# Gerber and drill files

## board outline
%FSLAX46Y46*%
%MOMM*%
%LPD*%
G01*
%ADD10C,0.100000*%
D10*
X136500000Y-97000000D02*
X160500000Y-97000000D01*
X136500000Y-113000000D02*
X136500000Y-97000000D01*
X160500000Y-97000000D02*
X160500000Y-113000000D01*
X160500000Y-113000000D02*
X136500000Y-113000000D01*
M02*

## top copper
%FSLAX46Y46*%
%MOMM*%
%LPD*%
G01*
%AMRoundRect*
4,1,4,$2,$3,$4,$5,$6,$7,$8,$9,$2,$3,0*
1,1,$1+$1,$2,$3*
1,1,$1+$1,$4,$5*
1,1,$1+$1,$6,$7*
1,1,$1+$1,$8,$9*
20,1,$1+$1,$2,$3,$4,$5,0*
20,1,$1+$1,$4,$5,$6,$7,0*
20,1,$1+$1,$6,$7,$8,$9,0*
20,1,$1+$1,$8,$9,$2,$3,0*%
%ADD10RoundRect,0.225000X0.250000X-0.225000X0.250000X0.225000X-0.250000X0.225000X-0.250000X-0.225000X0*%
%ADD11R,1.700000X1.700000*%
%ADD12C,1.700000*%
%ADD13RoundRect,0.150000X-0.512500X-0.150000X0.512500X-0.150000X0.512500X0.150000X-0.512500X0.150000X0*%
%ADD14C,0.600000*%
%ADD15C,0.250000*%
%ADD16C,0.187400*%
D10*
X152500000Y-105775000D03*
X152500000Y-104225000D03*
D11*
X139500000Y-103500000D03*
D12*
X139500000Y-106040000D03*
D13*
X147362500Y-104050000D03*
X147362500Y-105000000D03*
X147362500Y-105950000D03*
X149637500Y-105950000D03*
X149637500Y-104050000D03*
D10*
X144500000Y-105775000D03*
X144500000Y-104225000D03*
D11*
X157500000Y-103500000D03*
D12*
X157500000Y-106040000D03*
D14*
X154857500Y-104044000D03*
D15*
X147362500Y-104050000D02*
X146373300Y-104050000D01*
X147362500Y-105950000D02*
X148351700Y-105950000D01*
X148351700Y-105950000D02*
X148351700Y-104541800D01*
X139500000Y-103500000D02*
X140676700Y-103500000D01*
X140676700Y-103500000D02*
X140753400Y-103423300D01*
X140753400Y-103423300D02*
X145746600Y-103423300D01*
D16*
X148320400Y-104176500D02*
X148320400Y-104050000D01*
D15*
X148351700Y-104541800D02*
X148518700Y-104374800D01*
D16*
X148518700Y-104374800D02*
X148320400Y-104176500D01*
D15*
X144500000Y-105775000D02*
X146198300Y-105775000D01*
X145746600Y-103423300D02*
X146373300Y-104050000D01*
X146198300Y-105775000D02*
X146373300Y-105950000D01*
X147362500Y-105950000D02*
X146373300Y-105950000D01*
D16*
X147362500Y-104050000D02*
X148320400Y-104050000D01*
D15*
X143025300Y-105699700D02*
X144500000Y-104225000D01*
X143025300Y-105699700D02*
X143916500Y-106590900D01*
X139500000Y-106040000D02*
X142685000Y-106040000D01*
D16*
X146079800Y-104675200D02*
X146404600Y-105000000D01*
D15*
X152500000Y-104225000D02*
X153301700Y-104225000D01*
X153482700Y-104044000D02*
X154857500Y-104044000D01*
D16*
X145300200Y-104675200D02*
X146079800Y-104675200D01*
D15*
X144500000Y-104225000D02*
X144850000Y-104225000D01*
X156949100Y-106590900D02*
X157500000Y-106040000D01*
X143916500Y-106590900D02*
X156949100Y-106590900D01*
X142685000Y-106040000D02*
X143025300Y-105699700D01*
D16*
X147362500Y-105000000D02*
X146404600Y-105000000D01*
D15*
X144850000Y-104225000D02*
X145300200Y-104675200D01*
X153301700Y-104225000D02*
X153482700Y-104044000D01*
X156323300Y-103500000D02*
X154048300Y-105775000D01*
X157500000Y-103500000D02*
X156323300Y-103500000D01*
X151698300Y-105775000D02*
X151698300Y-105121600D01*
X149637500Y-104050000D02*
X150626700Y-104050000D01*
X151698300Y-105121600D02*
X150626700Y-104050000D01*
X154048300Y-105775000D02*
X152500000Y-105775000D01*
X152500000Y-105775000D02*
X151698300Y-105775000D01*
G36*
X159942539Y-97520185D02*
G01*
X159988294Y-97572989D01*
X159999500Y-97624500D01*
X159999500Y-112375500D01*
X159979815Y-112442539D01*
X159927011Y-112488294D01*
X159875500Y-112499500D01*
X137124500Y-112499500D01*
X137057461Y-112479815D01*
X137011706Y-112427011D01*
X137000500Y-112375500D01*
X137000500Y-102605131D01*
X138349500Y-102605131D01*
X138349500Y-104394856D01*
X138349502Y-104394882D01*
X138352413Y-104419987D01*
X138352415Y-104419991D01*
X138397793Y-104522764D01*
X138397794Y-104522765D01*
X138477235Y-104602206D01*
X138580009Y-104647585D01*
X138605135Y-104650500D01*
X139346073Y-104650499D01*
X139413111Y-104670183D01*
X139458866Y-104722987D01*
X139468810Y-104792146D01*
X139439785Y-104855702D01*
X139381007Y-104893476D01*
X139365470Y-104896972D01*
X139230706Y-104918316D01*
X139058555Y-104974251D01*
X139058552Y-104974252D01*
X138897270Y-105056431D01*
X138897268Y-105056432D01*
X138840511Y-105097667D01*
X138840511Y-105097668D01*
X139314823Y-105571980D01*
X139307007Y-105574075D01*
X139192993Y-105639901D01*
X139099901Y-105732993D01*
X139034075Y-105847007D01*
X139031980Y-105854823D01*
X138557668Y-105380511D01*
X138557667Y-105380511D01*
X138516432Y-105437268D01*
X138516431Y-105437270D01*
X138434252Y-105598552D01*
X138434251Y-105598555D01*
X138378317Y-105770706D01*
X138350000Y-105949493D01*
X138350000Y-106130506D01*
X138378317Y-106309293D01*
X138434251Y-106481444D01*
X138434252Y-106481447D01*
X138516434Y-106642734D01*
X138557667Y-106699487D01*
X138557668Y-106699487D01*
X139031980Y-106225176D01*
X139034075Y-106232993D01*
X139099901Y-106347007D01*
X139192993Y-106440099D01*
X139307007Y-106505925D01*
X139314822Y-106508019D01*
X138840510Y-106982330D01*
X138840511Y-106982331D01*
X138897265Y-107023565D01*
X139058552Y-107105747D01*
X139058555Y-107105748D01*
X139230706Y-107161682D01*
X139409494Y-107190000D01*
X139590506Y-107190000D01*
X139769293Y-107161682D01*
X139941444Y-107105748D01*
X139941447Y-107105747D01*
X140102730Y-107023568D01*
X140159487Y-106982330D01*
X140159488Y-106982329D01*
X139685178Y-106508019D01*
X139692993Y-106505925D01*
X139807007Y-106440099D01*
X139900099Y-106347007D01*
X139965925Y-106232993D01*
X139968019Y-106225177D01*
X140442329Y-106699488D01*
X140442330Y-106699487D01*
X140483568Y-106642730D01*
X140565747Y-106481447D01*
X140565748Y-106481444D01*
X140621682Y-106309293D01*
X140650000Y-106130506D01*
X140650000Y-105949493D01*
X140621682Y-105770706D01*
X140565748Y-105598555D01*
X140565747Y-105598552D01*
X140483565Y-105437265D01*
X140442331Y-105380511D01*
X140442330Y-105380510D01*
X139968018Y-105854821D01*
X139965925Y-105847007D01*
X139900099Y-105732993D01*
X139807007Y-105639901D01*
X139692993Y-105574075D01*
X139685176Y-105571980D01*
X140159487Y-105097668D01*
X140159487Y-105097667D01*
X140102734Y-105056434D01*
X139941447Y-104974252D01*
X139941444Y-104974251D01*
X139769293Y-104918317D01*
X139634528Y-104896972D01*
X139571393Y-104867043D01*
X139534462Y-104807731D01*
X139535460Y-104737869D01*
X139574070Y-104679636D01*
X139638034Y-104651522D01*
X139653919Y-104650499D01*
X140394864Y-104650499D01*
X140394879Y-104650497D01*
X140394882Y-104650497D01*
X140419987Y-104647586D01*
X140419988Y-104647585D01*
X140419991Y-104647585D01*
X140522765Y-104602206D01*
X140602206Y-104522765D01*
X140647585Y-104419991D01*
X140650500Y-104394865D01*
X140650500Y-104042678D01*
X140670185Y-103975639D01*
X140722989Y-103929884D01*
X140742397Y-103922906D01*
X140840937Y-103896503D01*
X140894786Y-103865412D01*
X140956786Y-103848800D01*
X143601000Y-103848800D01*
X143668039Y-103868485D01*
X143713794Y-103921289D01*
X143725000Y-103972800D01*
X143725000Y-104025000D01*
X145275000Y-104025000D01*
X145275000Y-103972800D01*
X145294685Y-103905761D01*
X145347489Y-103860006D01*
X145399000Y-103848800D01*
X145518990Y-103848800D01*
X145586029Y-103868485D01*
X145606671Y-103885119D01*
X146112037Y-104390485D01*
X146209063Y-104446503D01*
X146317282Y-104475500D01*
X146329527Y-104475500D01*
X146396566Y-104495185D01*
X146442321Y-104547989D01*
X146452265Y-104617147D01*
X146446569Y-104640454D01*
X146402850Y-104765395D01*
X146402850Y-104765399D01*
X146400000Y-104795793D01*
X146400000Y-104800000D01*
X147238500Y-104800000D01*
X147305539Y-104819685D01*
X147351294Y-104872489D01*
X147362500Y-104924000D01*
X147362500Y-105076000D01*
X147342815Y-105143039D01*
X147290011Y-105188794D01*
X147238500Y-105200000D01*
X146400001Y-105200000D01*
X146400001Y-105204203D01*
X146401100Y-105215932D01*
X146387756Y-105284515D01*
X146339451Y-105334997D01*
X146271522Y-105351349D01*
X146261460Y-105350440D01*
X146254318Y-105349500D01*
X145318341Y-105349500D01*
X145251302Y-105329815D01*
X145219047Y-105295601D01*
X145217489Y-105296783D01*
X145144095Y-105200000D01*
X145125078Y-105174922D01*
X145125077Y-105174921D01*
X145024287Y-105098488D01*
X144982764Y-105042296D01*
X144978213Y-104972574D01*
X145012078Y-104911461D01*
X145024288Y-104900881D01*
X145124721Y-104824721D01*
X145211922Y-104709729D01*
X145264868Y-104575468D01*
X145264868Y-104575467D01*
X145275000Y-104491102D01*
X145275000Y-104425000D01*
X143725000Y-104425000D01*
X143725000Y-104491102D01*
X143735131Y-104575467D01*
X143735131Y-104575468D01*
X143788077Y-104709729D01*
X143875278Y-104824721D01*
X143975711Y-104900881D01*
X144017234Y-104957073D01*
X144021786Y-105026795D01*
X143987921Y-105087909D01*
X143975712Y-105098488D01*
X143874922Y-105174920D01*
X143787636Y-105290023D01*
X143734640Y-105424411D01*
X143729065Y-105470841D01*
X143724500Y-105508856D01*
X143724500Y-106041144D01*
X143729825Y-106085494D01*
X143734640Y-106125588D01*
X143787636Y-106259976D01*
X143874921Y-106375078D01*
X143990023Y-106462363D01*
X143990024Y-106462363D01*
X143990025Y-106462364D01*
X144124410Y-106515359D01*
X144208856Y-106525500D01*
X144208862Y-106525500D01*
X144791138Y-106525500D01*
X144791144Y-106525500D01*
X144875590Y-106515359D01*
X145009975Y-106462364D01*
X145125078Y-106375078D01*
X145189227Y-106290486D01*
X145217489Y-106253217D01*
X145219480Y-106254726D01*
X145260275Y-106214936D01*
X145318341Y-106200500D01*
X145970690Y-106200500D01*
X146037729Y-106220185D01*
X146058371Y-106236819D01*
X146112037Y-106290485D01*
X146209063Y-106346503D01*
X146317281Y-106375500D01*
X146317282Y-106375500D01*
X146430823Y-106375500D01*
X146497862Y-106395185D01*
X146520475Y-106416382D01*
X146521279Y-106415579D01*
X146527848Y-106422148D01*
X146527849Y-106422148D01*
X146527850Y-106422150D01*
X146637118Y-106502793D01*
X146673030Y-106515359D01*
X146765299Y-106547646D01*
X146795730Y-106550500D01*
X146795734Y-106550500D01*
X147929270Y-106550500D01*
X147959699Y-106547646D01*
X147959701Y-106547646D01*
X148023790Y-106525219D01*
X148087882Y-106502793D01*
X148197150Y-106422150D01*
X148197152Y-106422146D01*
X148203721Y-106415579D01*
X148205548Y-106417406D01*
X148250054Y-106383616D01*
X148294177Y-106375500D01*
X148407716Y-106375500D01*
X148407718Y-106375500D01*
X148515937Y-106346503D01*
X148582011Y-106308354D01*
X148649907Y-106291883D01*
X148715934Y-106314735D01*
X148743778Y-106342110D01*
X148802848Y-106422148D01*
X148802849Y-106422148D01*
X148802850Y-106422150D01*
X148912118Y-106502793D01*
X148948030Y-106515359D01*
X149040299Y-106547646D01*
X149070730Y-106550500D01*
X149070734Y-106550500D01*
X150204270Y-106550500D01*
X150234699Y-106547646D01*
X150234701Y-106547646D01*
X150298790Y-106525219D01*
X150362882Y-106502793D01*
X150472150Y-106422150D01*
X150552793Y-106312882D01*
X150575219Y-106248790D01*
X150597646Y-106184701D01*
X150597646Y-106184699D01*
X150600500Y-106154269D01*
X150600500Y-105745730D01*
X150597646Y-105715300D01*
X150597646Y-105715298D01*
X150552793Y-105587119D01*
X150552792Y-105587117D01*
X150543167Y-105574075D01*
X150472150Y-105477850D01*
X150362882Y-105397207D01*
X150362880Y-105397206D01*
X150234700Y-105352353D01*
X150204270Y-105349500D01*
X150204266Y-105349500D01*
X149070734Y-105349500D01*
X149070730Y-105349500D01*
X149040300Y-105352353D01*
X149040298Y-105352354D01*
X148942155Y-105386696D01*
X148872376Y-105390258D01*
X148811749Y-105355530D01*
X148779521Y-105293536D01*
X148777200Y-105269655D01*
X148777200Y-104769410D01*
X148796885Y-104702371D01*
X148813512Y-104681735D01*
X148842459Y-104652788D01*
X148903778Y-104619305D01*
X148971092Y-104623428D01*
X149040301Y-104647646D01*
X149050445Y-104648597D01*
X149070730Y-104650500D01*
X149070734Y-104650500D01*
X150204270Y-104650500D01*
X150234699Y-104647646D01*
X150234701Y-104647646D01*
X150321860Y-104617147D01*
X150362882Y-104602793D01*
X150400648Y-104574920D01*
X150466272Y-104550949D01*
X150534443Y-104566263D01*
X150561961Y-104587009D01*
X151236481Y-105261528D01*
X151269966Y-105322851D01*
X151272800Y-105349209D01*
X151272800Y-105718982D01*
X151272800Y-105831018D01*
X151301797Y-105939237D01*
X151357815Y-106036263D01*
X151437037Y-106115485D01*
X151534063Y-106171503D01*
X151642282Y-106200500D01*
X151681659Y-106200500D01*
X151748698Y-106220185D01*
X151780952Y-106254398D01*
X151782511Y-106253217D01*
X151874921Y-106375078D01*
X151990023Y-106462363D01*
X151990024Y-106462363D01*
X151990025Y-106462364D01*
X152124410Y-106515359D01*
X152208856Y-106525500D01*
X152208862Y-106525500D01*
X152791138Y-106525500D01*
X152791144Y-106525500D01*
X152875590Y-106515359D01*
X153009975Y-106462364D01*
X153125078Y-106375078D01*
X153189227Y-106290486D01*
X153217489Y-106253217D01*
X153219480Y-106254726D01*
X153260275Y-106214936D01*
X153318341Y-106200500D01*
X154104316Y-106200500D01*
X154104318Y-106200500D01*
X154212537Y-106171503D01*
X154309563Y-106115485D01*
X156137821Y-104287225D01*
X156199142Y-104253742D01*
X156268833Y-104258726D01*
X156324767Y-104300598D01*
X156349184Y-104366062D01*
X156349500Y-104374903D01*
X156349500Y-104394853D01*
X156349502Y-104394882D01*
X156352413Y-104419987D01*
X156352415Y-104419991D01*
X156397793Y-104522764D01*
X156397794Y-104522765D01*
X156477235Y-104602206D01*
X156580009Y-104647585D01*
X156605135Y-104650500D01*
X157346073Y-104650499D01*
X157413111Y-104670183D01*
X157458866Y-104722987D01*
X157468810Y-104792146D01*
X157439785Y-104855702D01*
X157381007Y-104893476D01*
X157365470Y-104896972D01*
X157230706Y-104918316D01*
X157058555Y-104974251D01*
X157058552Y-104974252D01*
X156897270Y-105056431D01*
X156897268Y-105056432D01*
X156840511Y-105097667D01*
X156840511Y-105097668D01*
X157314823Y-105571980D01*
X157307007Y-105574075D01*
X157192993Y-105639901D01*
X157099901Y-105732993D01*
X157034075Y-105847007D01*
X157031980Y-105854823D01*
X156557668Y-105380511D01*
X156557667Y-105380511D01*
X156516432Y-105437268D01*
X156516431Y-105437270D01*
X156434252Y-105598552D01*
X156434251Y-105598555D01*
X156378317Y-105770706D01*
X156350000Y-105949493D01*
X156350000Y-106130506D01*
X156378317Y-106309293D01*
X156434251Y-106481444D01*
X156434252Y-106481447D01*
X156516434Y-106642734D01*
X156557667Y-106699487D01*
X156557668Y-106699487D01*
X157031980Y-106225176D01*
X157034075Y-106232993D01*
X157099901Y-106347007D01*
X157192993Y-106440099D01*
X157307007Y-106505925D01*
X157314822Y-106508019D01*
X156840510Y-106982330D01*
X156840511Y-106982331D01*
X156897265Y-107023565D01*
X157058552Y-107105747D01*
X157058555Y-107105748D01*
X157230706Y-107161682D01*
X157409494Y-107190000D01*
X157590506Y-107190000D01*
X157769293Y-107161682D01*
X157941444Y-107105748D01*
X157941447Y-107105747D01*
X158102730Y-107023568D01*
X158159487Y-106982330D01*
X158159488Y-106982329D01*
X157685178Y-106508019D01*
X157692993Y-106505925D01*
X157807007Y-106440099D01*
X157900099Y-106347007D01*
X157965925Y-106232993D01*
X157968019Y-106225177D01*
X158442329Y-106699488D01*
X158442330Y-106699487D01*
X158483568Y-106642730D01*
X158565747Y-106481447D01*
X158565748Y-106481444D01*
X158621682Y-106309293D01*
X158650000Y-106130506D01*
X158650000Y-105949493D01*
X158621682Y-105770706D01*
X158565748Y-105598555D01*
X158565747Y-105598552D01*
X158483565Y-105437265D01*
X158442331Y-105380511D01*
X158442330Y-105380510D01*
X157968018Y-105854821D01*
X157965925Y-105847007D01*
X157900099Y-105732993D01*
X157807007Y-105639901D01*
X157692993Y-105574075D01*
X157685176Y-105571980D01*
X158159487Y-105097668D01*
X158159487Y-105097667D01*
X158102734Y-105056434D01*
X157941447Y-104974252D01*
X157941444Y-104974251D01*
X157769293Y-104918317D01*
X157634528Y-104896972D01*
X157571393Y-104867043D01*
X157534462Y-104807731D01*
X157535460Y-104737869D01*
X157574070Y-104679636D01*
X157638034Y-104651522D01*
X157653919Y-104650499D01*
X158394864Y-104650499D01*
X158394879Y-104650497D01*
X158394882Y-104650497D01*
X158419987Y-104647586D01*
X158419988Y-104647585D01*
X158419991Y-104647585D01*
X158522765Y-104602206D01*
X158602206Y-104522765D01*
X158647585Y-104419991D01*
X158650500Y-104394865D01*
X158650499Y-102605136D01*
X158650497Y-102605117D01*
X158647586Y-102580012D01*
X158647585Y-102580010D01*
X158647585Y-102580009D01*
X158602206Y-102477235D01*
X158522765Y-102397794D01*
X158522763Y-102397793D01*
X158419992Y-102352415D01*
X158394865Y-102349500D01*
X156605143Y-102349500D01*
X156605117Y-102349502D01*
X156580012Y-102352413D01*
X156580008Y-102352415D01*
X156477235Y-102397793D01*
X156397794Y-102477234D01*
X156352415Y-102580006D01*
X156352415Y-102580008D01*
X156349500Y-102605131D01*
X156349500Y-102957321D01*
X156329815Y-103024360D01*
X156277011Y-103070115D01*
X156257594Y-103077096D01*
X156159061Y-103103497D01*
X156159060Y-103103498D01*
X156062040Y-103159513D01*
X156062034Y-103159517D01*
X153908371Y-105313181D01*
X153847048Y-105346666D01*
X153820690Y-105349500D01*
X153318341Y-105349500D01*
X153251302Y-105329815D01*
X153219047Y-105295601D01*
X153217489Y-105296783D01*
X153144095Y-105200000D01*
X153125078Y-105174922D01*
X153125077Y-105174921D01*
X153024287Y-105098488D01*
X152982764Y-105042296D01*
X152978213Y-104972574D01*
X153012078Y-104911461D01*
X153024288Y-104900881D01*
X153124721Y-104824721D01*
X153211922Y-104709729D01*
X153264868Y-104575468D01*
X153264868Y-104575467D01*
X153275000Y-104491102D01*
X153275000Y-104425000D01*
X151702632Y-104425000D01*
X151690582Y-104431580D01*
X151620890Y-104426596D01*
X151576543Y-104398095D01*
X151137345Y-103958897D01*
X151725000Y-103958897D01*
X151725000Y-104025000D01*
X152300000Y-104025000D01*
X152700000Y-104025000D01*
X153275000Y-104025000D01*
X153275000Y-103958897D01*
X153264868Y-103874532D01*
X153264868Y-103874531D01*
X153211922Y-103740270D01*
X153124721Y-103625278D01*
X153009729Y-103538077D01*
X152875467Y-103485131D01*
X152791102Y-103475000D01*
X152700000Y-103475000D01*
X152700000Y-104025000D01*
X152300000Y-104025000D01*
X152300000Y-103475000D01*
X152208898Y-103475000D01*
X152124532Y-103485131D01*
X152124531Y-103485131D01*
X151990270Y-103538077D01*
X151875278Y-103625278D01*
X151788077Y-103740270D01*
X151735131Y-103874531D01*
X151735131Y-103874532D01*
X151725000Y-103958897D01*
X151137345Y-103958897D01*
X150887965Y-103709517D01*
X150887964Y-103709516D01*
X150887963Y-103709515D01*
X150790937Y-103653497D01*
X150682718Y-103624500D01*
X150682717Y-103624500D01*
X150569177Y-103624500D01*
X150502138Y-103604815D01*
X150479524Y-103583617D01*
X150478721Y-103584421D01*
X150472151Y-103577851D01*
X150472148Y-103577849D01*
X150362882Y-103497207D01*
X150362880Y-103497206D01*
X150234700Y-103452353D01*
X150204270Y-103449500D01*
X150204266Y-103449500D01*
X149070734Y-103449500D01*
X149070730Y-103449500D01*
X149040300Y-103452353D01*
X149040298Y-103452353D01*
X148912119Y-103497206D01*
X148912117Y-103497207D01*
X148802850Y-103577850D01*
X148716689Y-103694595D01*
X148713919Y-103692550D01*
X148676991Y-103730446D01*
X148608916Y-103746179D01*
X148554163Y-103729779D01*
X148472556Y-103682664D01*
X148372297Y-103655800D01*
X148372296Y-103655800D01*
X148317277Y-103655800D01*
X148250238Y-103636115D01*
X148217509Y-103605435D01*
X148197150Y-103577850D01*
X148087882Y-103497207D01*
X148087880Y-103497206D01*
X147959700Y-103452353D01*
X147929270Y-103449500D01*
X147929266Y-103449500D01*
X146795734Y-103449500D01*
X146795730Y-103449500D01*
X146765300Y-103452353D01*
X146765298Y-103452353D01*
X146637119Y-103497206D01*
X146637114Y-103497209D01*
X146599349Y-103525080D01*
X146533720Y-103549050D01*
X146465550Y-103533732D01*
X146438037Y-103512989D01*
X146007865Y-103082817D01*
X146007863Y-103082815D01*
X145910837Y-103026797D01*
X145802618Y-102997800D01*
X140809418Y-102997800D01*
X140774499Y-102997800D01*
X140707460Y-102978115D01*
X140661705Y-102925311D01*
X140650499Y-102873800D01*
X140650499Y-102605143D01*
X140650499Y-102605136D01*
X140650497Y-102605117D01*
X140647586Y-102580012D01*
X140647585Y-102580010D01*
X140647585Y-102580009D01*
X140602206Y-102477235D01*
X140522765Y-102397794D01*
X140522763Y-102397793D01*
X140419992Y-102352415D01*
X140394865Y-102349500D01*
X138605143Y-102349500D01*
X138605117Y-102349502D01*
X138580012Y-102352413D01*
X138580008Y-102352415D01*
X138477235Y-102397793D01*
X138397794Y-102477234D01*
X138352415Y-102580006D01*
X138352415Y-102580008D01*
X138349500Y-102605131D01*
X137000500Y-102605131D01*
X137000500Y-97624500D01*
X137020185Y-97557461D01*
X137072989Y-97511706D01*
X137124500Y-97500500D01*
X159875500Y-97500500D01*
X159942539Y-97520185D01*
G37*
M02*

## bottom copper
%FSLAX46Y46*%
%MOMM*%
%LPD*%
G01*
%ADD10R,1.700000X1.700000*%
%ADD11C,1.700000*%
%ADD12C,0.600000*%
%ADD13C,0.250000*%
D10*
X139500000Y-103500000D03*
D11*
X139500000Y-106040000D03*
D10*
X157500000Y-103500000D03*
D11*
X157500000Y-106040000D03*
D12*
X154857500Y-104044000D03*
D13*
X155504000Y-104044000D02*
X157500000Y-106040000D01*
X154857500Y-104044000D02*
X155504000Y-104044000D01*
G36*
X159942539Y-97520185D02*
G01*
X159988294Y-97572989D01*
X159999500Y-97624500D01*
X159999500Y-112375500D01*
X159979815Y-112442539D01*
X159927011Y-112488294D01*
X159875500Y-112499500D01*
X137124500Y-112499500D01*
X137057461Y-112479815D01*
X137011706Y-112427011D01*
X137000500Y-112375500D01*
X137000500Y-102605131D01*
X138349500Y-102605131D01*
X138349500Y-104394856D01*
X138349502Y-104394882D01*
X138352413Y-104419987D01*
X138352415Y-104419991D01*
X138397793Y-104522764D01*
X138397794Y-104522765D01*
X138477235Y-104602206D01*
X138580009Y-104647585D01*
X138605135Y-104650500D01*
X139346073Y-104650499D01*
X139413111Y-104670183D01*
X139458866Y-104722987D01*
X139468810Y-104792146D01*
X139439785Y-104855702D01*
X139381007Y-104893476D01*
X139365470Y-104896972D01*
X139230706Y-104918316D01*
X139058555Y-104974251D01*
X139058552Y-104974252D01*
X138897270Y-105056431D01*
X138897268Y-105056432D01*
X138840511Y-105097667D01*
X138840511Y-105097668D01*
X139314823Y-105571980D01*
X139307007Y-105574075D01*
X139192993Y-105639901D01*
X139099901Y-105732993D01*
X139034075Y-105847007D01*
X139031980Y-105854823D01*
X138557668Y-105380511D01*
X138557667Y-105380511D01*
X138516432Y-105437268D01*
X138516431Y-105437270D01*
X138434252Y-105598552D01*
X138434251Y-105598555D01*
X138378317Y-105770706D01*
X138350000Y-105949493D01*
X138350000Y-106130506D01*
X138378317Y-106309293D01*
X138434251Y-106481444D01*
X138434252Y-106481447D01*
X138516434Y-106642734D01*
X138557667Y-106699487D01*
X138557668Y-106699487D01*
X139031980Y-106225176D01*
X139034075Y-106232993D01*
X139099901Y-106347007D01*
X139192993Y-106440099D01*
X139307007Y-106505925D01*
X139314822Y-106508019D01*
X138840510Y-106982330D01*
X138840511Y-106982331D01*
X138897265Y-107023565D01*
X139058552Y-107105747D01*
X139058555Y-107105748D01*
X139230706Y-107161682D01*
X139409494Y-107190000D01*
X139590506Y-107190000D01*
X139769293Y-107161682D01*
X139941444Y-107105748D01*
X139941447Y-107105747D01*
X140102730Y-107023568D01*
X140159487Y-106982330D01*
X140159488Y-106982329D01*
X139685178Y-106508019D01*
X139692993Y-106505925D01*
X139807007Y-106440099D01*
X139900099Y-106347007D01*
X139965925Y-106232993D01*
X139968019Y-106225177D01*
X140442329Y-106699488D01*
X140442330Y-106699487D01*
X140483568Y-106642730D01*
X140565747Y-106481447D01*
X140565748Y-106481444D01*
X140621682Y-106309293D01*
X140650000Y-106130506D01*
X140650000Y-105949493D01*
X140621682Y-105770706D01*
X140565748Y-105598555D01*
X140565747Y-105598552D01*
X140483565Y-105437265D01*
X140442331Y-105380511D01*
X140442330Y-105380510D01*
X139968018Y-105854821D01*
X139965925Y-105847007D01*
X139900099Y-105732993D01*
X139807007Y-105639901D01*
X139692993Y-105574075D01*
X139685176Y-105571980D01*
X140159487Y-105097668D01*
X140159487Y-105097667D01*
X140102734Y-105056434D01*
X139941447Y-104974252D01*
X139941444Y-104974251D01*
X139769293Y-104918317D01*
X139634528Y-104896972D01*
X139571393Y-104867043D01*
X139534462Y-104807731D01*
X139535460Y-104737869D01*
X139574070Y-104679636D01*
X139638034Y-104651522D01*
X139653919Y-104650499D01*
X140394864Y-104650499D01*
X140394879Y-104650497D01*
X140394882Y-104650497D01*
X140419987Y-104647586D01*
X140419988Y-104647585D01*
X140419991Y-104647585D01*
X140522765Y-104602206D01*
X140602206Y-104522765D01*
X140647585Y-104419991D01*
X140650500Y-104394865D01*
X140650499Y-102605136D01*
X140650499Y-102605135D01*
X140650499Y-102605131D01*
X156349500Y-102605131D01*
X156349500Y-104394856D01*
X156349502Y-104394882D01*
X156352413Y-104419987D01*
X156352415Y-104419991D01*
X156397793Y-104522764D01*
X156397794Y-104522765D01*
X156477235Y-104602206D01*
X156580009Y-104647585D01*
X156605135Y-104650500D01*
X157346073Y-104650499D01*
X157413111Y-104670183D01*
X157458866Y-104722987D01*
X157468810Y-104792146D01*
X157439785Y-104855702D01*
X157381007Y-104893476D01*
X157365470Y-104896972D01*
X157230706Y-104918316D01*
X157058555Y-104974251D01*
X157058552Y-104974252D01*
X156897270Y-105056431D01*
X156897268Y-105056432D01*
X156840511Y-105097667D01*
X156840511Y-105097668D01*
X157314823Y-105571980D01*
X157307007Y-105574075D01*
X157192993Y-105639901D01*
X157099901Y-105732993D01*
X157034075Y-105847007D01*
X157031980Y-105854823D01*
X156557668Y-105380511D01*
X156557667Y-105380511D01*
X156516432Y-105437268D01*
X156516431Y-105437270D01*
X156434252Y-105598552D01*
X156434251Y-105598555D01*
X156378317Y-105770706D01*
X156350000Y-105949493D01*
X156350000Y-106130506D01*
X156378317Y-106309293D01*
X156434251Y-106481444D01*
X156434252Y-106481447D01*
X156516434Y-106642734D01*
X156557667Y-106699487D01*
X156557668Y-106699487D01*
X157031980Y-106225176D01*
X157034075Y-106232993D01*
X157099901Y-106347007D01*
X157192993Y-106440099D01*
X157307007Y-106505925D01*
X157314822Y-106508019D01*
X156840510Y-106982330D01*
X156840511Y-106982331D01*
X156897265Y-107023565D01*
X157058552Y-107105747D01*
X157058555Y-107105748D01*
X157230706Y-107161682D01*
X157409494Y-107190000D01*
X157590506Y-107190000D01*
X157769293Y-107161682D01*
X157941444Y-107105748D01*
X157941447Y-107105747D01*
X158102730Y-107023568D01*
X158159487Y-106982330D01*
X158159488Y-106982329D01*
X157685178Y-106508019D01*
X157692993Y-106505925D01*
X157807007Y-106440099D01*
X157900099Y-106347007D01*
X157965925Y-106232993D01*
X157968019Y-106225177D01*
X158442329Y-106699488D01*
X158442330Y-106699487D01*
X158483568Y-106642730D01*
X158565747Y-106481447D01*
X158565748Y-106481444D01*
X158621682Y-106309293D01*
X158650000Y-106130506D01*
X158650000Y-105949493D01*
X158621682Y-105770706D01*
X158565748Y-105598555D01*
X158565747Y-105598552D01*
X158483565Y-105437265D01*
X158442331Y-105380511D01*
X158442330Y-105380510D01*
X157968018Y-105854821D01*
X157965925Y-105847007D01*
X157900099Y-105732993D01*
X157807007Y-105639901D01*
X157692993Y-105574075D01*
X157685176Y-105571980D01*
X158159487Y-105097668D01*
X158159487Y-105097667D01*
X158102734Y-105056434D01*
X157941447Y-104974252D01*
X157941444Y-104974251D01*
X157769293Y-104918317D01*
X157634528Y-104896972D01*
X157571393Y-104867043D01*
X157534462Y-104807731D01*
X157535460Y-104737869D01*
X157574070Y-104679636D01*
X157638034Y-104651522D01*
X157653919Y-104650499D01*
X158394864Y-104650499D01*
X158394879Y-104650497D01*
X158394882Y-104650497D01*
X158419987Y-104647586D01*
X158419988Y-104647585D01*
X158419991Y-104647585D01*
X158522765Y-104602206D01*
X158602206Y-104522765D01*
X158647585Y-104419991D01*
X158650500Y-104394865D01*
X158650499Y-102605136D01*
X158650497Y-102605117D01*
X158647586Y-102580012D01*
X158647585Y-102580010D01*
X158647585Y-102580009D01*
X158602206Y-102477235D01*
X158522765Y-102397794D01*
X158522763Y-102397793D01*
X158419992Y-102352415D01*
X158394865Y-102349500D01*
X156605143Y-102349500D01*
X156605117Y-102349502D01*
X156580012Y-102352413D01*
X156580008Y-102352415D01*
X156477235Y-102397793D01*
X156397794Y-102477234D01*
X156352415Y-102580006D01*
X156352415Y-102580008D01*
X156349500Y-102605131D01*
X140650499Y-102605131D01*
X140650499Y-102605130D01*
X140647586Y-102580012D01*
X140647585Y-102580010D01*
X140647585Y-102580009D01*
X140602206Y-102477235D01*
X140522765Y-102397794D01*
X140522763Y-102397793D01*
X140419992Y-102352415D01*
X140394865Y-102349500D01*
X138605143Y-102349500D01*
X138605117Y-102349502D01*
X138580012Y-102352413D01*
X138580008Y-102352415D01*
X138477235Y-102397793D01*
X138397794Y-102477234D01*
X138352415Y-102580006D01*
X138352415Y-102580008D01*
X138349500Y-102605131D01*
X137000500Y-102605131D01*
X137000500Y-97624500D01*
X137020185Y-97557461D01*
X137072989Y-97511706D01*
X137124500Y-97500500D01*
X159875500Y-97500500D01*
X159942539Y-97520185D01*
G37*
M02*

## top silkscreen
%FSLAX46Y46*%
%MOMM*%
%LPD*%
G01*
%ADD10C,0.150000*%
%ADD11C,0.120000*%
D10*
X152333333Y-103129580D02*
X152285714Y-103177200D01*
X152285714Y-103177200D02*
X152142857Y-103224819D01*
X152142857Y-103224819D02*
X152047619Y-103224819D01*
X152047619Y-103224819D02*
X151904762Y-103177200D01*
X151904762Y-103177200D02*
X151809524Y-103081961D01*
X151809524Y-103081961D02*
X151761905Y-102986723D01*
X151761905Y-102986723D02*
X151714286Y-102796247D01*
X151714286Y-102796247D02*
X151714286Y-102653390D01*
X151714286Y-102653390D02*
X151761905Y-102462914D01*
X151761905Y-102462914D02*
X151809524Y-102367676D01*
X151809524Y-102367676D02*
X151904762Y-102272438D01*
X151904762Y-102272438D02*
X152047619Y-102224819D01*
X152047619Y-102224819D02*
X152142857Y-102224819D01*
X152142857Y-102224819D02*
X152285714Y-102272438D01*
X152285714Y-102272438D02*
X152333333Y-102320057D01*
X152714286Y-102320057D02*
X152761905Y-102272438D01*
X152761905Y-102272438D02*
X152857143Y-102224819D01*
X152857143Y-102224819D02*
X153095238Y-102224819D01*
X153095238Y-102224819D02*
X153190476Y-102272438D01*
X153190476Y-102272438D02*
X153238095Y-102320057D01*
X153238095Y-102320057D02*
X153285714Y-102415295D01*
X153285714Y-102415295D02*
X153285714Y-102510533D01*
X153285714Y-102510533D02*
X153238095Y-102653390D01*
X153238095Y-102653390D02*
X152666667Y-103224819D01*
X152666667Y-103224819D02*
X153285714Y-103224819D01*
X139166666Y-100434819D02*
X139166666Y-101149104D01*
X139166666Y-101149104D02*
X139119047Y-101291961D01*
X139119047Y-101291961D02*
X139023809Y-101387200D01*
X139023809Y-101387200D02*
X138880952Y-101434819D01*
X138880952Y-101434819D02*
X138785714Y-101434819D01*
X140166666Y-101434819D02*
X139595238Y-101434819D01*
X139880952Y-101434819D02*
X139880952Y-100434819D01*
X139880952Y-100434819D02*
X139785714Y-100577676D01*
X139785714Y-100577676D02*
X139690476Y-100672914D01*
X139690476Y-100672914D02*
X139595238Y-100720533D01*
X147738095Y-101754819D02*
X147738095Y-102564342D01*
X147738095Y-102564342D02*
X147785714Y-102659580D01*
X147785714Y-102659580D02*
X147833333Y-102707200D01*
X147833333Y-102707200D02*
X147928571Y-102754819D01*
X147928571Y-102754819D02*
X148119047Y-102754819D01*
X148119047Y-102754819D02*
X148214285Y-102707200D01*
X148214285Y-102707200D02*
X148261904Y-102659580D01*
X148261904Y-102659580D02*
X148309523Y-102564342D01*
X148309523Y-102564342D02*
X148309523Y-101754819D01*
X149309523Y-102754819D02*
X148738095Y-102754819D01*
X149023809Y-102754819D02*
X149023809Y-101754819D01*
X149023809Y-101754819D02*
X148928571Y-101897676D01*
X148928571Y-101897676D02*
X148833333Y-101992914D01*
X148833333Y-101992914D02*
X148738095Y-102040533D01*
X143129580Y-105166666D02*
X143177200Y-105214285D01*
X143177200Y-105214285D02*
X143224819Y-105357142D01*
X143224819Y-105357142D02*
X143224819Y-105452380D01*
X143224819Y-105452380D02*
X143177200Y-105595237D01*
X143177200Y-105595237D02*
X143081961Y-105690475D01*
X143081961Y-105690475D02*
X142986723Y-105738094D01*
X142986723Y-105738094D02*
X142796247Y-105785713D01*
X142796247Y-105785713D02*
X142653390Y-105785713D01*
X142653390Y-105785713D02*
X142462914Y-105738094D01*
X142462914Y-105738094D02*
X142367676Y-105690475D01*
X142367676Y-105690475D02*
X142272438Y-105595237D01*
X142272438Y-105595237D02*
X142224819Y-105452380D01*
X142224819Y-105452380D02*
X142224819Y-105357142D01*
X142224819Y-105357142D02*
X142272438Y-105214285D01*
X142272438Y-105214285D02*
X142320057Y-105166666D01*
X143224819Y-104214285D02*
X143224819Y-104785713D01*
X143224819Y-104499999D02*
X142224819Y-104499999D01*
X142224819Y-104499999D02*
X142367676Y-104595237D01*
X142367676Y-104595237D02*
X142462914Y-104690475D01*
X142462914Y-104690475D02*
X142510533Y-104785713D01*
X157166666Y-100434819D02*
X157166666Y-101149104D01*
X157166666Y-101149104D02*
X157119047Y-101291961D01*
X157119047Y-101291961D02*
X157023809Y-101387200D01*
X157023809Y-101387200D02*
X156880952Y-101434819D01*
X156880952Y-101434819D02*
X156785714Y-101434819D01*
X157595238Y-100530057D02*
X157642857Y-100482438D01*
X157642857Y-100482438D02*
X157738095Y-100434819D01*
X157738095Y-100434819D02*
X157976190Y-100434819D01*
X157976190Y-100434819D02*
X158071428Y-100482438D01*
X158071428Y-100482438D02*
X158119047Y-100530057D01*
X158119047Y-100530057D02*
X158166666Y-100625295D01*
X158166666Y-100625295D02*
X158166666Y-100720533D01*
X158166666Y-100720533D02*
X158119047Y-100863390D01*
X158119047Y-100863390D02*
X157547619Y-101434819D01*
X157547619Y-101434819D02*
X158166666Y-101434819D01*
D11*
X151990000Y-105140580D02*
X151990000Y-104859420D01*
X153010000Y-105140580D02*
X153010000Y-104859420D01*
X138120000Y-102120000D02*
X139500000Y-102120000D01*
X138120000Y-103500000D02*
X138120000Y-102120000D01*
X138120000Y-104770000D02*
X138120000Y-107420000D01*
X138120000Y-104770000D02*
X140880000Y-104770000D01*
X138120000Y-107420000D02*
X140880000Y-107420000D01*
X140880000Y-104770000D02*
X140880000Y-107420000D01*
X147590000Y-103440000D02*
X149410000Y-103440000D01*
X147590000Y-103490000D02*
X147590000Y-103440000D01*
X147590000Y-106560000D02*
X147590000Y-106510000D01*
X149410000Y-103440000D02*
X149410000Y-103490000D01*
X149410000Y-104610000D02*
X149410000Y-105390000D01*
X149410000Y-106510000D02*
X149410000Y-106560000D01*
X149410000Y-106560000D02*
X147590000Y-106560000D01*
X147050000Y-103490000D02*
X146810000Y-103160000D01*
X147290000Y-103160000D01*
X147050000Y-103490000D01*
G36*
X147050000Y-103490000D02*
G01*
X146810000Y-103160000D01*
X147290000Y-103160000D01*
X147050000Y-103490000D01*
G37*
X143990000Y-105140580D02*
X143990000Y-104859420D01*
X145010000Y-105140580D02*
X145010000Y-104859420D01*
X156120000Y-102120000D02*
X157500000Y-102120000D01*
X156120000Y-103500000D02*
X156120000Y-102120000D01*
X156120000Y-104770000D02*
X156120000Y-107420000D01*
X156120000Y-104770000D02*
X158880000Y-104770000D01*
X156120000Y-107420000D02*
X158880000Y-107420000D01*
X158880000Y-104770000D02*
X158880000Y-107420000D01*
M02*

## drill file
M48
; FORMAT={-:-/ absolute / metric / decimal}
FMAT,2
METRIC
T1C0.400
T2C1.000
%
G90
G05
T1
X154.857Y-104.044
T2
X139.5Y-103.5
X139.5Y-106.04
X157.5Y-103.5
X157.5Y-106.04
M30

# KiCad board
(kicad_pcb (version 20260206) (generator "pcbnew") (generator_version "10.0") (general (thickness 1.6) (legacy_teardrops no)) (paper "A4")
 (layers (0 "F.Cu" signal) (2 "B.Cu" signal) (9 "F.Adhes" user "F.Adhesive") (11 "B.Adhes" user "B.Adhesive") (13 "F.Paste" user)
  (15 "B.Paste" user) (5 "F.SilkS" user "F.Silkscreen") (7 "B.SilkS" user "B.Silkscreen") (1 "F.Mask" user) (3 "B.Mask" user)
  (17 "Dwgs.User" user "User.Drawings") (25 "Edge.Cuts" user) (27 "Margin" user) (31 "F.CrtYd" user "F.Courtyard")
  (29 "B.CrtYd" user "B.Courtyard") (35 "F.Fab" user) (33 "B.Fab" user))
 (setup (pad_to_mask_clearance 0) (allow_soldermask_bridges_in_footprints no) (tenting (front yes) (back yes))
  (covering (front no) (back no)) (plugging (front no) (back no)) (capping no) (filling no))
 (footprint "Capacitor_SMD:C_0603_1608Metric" (layer "F.Cu") (at 152.5 105 90)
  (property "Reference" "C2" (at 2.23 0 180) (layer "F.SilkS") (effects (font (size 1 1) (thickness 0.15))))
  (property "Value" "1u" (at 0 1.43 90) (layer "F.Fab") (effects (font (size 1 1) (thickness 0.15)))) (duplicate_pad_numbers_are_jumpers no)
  (fp_line (start -0.14058 -0.51) (end 0.14058 -0.51) (stroke (width 0.12) (type solid)) (layer "F.SilkS"))
  (fp_line (start -0.14058 0.51) (end 0.14058 0.51) (stroke (width 0.12) (type solid)) (layer "F.SilkS"))
  (pad "1" smd roundrect (at -0.775 0 90) (size 0.9 0.95) (layers "F.Cu" "F.Mask" "F.Paste") (roundrect_rratio 0.25) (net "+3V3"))
  (pad "2" smd roundrect (at 0.775 0 90) (size 0.9 0.95) (layers "F.Cu" "F.Mask" "F.Paste") (roundrect_rratio 0.25) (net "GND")))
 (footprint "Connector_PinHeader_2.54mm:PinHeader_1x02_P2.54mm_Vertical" (layer "F.Cu") (at 139.5 103.5)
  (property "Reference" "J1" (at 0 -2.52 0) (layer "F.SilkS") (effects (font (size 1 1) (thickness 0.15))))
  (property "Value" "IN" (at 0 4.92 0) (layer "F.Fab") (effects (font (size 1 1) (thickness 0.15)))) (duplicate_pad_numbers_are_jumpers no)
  (fp_line (start -1.38 -1.38) (end 0 -1.38) (stroke (width 0.12) (type solid)) (layer "F.SilkS"))
  (fp_line (start -1.38 0) (end -1.38 -1.38) (stroke (width 0.12) (type solid)) (layer "F.SilkS"))
  (fp_line (start -1.38 1.27) (end -1.38 3.92) (stroke (width 0.12) (type solid)) (layer "F.SilkS"))
  (fp_line (start -1.38 1.27) (end 1.38 1.27) (stroke (width 0.12) (type solid)) (layer "F.SilkS"))
  (fp_line (start -1.38 3.92) (end 1.38 3.92) (stroke (width 0.12) (type solid)) (layer "F.SilkS"))
  (fp_line (start 1.38 1.27) (end 1.38 3.92) (stroke (width 0.12) (type solid)) (layer "F.SilkS"))
  (pad "1" thru_hole rect (at 0 0) (size 1.7 1.7) (drill 1) (layers "*.Cu" "*.Mask") (remove_unused_layers no) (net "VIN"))
  (pad "2" thru_hole circle (at 0 2.54) (size 1.7 1.7) (drill 1) (layers "*.Cu" "*.Mask") (remove_unused_layers no) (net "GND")))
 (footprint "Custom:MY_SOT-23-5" (layer "F.Cu") (at 148.5 105)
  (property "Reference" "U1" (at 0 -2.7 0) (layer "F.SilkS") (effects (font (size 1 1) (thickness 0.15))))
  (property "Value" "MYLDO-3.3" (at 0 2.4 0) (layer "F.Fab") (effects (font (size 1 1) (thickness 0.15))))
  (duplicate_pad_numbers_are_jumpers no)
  (fp_line (start -0.91 -1.56) (end 0.91 -1.56) (stroke (width 0.12) (type solid)) (layer "F.SilkS"))
  (fp_line (start -0.91 -1.51) (end -0.91 -1.56) (stroke (width 0.12) (type solid)) (layer "F.SilkS"))
  (fp_line (start -0.91 1.56) (end -0.91 1.51) (stroke (width 0.12) (type solid)) (layer "F.SilkS"))
  (fp_line (start 0.91 -1.56) (end 0.91 -1.51) (stroke (width 0.12) (type solid)) (layer "F.SilkS"))
  (fp_line (start 0.91 -0.39) (end 0.91 0.39) (stroke (width 0.12) (type solid)) (layer "F.SilkS"))
  (fp_line (start 0.91 1.51) (end 0.91 1.56) (stroke (width 0.12) (type solid)) (layer "F.SilkS"))
  (fp_line (start 0.91 1.56) (end -0.91 1.56) (stroke (width 0.12) (type solid)) (layer "F.SilkS"))
  (fp_poly (pts (xy -1.45 -1.51) (xy -1.69 -1.84) (xy -1.21 -1.84)) (stroke (width 0.12) (type solid)) (fill yes) (layer "F.SilkS"))
  (pad "1" smd roundrect (at -1.1375 -0.95) (size 1.325 0.6) (layers "F.Cu" "F.Mask" "F.Paste") (roundrect_rratio 0.25) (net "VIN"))
  (pad "2" smd roundrect (at -1.1375 0) (size 1.325 0.6) (layers "F.Cu" "F.Mask" "F.Paste") (roundrect_rratio 0.25) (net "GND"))
  (pad "3" smd roundrect (at -1.1375 0.95) (size 1.325 0.6) (layers "F.Cu" "F.Mask" "F.Paste") (roundrect_rratio 0.25) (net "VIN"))
  (pad "4" smd roundrect (at 1.1375 0.95) (size 1.325 0.6) (layers "F.Cu" "F.Mask" "F.Paste") (roundrect_rratio 0.25)
   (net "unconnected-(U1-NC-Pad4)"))
  (pad "5" smd roundrect (at 1.1375 -0.95) (size 1.325 0.6) (layers "F.Cu" "F.Mask" "F.Paste") (roundrect_rratio 0.25) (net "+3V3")))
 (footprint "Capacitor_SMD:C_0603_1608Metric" (layer "F.Cu") (at 144.5 105 90)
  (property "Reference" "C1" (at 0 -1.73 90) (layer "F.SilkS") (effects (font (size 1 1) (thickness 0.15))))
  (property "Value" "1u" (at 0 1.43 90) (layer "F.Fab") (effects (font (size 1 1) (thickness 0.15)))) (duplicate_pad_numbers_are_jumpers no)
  (fp_line (start -0.14058 -0.51) (end 0.14058 -0.51) (stroke (width 0.12) (type solid)) (layer "F.SilkS"))
  (fp_line (start -0.14058 0.51) (end 0.14058 0.51) (stroke (width 0.12) (type solid)) (layer "F.SilkS"))
  (pad "1" smd roundrect (at -0.775 0 90) (size 0.9 0.95) (layers "F.Cu" "F.Mask" "F.Paste") (roundrect_rratio 0.25) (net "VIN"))
  (pad "2" smd roundrect (at 0.775 0 90) (size 0.9 0.95) (layers "F.Cu" "F.Mask" "F.Paste") (roundrect_rratio 0.25) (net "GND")))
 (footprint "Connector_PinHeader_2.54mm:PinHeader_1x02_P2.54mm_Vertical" (layer "F.Cu") (at 157.5 103.5)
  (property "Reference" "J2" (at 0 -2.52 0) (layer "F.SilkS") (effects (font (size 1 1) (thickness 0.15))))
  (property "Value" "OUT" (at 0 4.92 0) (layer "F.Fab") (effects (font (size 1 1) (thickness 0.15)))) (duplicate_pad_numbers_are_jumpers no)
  (fp_line (start -1.38 -1.38) (end 0 -1.38) (stroke (width 0.12) (type solid)) (layer "F.SilkS"))
  (fp_line (start -1.38 0) (end -1.38 -1.38) (stroke (width 0.12) (type solid)) (layer "F.SilkS"))
  (fp_line (start -1.38 1.27) (end -1.38 3.92) (stroke (width 0.12) (type solid)) (layer "F.SilkS"))
  (fp_line (start -1.38 1.27) (end 1.38 1.27) (stroke (width 0.12) (type solid)) (layer "F.SilkS"))
  (fp_line (start -1.38 3.92) (end 1.38 3.92) (stroke (width 0.12) (type solid)) (layer "F.SilkS"))
  (fp_line (start 1.38 1.27) (end 1.38 3.92) (stroke (width 0.12) (type solid)) (layer "F.SilkS"))
  (pad "1" thru_hole rect (at 0 0) (size 1.7 1.7) (drill 1) (layers "*.Cu" "*.Mask") (remove_unused_layers no) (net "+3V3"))
  (pad "2" thru_hole circle (at 0 2.54) (size 1.7 1.7) (drill 1) (layers "*.Cu" "*.Mask") (remove_unused_layers no) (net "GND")))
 (gr_line (start 136.5 97) (end 160.5 97) (stroke (width 0.1) (type default)) (layer "Edge.Cuts"))
 (gr_line (start 136.5 113) (end 136.5 97) (stroke (width 0.1) (type default)) (layer "Edge.Cuts"))
 (gr_line (start 160.5 97) (end 160.5 113) (stroke (width 0.1) (type default)) (layer "Edge.Cuts"))
 (gr_line (start 160.5 113) (end 136.5 113) (stroke (width 0.1) (type default)) (layer "Edge.Cuts"))
 (segment (start 147.3625 104.05) (end 146.3733 104.05) (width 0.25) (layer "F.Cu") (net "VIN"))
 (segment (start 147.3625 105.95) (end 148.3517 105.95) (width 0.25) (layer "F.Cu") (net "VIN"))
 (segment (start 148.3517 105.95) (end 148.3517 104.5418) (width 0.25) (layer "F.Cu") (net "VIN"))
 (segment (start 139.5 103.5) (end 140.6767 103.5) (width 0.25) (layer "F.Cu") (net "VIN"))
 (segment (start 140.6767 103.5) (end 140.7534 103.4233) (width 0.25) (layer "F.Cu") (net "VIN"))
 (segment (start 140.7534 103.4233) (end 145.7466 103.4233) (width 0.25) (layer "F.Cu") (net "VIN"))
 (segment (start 148.3204 104.1765) (end 148.3204 104.05) (width 0.1874) (layer "F.Cu") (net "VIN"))
 (segment (start 148.3517 104.5418) (end 148.5187 104.3748) (width 0.25) (layer "F.Cu") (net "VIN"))
 (segment (start 148.5187 104.3748) (end 148.3204 104.1765) (width 0.1874) (layer "F.Cu") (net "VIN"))
 (segment (start 144.5 105.775) (end 146.1983 105.775) (width 0.25) (layer "F.Cu") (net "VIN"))
 (segment (start 145.7466 103.4233) (end 146.3733 104.05) (width 0.25) (layer "F.Cu") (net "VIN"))
 (segment (start 146.1983 105.775) (end 146.3733 105.95) (width 0.25) (layer "F.Cu") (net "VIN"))
 (segment (start 147.3625 105.95) (end 146.3733 105.95) (width 0.25) (layer "F.Cu") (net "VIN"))
 (segment (start 147.3625 104.05) (end 148.3204 104.05) (width 0.1874) (layer "F.Cu") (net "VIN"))
 (segment (start 143.0253 105.6997) (end 144.5 104.225) (width 0.25) (layer "F.Cu") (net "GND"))
 (segment (start 143.0253 105.6997) (end 143.9165 106.5909) (width 0.25) (layer "F.Cu") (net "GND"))
 (segment (start 139.5 106.04) (end 142.685 106.04) (width 0.25) (layer "F.Cu") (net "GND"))
 (segment (start 146.0798 104.6752) (end 146.4046 105) (width 0.1874) (layer "F.Cu") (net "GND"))
 (segment (start 152.5 104.225) (end 153.3017 104.225) (width 0.25) (layer "F.Cu") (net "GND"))
 (segment (start 153.4827 104.044) (end 154.8575 104.044) (width 0.25) (layer "F.Cu") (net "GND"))
 (segment (start 145.3002 104.6752) (end 146.0798 104.6752) (width 0.1874) (layer "F.Cu") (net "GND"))
 (segment (start 144.5 104.225) (end 144.85 104.225) (width 0.25) (layer "F.Cu") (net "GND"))
 (segment (start 156.9491 106.5909) (end 157.5 106.04) (width 0.25) (layer "F.Cu") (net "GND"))
 (segment (start 143.9165 106.5909) (end 156.9491 106.5909) (width 0.25) (layer "F.Cu") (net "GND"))
 (segment (start 142.685 106.04) (end 143.0253 105.6997) (width 0.25) (layer "F.Cu") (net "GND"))
 (segment (start 147.3625 105) (end 146.4046 105) (width 0.1874) (layer "F.Cu") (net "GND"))
 (segment (start 144.85 104.225) (end 145.3002 104.6752) (width 0.25) (layer "F.Cu") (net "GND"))
 (segment (start 153.3017 104.225) (end 153.4827 104.044) (width 0.25) (layer "F.Cu") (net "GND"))
 (via (at 154.8575 104.044) (size 0.6) (drill 0.4) (layers "F.Cu" "B.Cu") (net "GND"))
 (segment (start 155.504 104.044) (end 157.5 106.04) (width 0.25) (layer "B.Cu") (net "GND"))
 (segment (start 154.8575 104.044) (end 155.504 104.044) (width 0.25) (layer "B.Cu") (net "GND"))
 (segment (start 156.3233 103.5) (end 154.0483 105.775) (width 0.25) (layer "F.Cu") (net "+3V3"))
 (segment (start 157.5 103.5) (end 156.3233 103.5) (width 0.25) (layer "F.Cu") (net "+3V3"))
 (segment (start 151.6983 105.775) (end 151.6983 105.1216) (width 0.25) (layer "F.Cu") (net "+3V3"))
 (segment (start 149.6375 104.05) (end 150.6267 104.05) (width 0.25) (layer "F.Cu") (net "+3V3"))
 (segment (start 151.6983 105.1216) (end 150.6267 104.05) (width 0.25) (layer "F.Cu") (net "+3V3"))
 (segment (start 154.0483 105.775) (end 152.5 105.775) (width 0.25) (layer "F.Cu") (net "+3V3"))
 (segment (start 152.5 105.775) (end 151.6983 105.775) (width 0.25) (layer "F.Cu") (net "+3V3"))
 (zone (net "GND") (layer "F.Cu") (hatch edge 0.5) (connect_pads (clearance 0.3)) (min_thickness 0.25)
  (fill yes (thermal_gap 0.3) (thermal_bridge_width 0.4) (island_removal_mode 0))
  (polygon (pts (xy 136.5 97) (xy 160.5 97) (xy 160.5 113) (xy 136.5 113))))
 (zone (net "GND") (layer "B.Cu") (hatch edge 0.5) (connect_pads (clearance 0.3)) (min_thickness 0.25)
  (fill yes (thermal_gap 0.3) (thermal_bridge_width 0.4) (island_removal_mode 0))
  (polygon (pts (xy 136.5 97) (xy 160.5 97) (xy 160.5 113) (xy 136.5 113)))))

